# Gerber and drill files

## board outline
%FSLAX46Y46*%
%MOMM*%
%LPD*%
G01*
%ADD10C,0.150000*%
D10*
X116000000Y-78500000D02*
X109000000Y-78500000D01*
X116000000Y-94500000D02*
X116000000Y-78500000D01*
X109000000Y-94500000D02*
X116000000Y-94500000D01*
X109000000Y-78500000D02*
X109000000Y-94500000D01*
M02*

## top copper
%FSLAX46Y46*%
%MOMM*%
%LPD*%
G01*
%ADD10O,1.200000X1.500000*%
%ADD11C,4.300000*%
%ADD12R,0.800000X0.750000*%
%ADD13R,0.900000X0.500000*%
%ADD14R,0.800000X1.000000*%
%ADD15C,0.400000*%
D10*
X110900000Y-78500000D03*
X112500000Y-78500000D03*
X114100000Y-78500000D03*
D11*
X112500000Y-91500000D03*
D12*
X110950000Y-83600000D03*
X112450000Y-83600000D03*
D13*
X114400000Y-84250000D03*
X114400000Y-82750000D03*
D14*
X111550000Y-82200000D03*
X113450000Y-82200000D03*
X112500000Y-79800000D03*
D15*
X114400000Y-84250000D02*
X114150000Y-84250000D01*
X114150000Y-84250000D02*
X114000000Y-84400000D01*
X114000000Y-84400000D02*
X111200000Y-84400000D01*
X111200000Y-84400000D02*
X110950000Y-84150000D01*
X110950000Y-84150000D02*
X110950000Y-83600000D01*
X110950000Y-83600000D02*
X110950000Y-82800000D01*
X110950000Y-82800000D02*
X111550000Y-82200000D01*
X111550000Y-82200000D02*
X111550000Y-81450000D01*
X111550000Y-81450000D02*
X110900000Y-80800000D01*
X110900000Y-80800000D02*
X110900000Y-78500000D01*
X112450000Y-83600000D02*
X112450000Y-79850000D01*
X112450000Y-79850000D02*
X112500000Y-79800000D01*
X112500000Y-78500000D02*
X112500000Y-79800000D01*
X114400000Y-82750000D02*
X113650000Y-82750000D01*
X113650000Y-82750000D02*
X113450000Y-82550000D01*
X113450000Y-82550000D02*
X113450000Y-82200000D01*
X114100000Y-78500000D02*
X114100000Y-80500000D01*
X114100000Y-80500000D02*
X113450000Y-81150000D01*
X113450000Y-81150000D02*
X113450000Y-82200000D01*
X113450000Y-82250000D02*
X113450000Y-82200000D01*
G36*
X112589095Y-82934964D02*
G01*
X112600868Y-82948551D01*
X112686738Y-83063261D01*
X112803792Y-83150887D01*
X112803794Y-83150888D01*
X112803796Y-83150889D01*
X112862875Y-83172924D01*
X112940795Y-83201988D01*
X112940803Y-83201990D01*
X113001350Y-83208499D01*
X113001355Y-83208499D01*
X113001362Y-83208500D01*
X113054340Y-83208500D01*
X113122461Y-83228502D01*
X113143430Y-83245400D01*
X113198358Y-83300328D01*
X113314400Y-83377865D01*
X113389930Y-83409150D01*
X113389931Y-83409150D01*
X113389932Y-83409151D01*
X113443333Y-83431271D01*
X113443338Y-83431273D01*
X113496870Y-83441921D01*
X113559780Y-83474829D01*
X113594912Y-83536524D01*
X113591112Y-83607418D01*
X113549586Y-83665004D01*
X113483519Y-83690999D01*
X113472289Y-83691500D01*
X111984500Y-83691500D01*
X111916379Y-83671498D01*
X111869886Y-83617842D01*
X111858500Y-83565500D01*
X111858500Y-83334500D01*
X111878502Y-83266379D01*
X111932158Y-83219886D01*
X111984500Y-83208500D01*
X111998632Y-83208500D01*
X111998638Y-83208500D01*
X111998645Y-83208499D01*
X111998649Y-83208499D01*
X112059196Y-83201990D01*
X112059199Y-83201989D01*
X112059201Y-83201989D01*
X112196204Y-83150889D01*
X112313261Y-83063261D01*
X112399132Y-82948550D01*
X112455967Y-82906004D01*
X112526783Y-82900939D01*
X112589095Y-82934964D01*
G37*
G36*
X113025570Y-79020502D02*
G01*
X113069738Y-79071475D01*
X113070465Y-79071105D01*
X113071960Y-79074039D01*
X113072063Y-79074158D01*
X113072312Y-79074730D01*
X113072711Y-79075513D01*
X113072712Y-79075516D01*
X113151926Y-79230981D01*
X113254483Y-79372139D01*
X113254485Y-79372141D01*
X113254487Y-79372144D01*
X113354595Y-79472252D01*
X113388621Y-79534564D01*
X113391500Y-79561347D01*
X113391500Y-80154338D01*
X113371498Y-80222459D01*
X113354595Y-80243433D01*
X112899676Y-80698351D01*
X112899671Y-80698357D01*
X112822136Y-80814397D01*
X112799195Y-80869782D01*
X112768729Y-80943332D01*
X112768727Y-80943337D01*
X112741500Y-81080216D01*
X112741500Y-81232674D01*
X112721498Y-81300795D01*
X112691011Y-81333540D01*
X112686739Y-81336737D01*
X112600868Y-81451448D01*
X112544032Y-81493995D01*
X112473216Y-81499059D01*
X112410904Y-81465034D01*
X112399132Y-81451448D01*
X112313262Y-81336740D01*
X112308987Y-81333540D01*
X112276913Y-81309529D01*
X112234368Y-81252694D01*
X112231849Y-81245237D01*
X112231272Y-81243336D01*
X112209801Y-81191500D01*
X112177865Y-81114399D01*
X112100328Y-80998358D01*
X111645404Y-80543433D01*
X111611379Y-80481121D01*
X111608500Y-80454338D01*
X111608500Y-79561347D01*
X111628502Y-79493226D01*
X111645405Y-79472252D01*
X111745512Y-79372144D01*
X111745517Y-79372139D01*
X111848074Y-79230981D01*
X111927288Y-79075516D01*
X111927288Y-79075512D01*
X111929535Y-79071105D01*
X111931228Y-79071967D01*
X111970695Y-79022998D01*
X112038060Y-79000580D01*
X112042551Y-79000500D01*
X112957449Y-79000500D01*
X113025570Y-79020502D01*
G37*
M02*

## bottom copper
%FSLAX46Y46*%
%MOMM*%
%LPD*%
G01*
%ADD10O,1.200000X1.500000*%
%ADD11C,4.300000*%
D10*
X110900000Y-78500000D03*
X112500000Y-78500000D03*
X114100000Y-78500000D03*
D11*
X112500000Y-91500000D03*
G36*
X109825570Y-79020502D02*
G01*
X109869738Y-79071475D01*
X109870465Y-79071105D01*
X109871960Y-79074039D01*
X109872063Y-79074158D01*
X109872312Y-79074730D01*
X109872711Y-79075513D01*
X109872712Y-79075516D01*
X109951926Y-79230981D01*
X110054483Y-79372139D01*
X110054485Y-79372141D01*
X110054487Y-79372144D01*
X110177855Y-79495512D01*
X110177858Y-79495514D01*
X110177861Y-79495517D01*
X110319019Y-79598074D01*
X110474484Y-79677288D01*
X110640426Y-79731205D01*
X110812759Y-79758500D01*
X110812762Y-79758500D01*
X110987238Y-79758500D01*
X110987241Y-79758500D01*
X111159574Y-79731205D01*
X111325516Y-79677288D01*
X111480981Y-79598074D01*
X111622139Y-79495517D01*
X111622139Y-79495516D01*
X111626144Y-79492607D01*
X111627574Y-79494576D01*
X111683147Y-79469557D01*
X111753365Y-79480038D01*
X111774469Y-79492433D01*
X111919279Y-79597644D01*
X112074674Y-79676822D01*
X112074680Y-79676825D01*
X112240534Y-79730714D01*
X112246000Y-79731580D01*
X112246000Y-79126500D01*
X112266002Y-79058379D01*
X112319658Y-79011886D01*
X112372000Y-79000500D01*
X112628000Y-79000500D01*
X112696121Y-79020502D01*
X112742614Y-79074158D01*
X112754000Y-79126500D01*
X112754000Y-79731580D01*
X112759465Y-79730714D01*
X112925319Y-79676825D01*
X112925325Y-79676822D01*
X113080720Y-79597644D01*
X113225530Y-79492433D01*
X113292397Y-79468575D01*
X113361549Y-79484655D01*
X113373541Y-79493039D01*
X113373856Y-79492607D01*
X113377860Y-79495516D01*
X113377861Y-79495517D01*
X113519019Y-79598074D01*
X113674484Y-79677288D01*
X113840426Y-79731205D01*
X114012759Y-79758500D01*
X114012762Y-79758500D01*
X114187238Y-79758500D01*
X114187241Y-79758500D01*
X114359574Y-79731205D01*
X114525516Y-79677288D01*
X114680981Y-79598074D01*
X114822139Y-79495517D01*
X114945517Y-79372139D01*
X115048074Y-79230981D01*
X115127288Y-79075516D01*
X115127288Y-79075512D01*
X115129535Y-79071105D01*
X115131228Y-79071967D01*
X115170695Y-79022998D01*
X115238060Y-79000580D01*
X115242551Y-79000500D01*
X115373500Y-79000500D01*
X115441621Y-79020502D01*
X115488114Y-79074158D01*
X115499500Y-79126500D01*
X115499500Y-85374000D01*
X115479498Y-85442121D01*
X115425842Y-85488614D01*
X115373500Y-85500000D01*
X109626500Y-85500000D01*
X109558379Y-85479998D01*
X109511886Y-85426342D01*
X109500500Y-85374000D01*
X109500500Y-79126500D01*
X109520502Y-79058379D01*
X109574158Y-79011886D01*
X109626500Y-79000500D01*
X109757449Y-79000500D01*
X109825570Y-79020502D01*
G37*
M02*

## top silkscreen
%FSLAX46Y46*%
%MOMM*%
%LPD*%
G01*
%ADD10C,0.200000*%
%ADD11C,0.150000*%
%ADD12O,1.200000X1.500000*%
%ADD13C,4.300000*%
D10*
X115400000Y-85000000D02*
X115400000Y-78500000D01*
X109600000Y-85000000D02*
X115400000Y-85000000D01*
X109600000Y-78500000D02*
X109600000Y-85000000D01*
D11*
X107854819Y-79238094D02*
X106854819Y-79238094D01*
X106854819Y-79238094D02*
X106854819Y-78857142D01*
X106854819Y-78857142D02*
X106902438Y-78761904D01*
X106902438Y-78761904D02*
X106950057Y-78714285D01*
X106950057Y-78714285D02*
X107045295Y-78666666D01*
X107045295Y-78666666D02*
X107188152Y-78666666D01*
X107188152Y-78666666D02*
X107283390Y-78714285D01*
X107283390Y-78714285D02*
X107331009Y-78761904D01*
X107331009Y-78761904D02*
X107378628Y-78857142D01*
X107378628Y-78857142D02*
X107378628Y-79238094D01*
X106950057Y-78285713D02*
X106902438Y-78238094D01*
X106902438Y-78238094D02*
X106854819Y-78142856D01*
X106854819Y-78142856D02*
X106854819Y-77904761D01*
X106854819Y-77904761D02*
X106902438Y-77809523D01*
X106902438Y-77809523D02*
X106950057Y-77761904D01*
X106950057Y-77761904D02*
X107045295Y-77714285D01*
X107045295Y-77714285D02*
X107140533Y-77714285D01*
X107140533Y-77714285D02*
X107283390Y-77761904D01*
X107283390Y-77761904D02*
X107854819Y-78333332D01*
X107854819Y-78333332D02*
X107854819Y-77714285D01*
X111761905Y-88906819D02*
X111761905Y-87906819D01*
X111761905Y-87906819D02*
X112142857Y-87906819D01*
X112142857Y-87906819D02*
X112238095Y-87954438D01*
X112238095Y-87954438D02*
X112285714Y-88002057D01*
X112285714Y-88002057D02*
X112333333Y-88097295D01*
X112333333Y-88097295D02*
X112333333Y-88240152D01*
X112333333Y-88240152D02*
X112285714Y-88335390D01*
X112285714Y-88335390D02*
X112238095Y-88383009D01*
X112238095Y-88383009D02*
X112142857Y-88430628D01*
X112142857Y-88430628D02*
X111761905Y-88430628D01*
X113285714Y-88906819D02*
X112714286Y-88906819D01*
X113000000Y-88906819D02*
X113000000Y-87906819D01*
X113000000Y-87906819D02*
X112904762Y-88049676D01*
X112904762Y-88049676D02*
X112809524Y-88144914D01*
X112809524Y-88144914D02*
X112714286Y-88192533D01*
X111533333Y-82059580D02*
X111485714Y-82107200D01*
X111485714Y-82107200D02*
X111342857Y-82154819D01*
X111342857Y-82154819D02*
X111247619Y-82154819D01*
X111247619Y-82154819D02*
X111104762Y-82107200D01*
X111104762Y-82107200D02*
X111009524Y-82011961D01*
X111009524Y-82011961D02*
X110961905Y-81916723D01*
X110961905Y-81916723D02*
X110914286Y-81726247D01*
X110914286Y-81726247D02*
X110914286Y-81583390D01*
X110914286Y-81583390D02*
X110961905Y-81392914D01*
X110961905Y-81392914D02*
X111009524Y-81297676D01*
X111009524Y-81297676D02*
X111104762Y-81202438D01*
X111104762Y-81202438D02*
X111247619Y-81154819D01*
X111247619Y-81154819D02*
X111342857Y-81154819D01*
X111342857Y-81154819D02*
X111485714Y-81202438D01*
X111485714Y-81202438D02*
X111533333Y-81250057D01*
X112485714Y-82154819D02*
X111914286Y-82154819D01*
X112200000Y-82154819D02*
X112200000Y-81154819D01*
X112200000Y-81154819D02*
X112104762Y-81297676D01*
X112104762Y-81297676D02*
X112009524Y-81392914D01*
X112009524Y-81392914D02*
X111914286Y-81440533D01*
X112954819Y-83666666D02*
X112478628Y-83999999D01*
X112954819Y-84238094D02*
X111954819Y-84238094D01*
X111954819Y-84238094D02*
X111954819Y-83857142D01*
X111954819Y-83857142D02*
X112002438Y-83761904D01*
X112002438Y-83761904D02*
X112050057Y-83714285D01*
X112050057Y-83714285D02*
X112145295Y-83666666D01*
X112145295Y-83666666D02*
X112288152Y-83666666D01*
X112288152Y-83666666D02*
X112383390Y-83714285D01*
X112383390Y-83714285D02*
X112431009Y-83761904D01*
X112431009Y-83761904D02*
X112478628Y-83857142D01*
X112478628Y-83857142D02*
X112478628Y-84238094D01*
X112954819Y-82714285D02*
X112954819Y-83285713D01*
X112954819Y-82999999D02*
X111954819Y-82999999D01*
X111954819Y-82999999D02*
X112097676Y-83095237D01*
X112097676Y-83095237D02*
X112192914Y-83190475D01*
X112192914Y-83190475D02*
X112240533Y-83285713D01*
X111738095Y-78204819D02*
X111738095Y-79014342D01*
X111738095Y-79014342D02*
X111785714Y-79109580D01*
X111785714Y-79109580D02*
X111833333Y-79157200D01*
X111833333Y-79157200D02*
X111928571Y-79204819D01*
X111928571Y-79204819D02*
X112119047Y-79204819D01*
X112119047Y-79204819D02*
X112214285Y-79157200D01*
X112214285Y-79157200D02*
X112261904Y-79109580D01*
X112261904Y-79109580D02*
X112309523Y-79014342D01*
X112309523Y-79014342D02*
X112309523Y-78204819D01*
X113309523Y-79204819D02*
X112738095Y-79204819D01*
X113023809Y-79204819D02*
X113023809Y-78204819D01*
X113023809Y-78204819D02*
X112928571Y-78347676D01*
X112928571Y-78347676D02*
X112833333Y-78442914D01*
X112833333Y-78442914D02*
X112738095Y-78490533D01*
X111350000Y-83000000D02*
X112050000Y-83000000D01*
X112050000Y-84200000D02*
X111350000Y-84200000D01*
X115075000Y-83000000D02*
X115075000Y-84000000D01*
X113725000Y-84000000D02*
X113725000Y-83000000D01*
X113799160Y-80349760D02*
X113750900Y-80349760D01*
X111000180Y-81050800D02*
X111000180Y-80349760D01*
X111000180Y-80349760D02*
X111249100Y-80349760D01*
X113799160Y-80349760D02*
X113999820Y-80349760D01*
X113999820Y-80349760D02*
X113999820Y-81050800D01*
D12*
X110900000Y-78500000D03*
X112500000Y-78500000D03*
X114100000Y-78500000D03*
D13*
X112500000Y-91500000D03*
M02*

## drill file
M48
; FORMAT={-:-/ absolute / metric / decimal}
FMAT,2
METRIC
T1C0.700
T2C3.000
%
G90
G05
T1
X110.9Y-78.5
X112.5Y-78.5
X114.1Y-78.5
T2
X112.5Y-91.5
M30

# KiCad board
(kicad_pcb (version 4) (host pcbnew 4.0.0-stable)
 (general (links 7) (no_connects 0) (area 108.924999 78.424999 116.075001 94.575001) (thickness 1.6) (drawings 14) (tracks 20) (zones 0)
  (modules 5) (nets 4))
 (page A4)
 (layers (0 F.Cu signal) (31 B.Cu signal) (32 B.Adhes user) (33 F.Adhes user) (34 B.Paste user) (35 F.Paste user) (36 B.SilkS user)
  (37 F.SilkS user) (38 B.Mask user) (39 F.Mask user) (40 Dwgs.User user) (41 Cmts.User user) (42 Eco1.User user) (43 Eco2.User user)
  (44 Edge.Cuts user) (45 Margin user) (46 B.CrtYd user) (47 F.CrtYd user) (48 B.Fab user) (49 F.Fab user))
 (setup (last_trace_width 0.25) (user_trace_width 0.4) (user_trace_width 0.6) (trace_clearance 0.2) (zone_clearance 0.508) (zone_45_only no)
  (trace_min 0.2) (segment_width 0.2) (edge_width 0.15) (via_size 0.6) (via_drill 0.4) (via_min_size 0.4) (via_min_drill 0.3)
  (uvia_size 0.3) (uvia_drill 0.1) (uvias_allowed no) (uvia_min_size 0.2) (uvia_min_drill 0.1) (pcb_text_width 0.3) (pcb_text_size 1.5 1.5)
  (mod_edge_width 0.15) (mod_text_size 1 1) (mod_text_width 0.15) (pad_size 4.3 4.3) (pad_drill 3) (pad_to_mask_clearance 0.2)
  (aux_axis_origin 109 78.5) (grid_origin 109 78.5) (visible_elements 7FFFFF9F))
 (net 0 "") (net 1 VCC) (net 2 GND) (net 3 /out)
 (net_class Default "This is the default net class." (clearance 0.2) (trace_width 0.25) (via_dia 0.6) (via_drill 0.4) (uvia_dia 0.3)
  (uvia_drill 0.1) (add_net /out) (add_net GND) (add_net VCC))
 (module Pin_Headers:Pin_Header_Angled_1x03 (layer F.Cu) (at 112.5 78.5 90)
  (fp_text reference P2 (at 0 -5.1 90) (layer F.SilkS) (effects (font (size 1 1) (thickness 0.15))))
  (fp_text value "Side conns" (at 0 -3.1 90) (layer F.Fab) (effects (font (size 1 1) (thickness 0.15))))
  (pad 1 thru_hole oval (at 0 -1.6 90) (size 1.5 1.2) (drill 0.7) (layers *.Cu *.Mask F.SilkS) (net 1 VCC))
  (pad 2 thru_hole oval (at 0 0 90) (size 1.5 1.2) (drill 0.7) (layers *.Cu *.Mask F.SilkS) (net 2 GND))
  (pad 3 thru_hole oval (at 0 1.6 90) (size 1.5 1.2) (drill 0.7) (layers *.Cu *.Mask F.SilkS) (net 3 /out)))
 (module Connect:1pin (layer F.Cu) (at 112.5 91.5)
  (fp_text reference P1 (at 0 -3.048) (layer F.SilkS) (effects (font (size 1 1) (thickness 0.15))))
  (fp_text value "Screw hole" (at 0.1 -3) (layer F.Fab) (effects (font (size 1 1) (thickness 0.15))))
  (pad 1 thru_hole circle (at 0 0) (size 4.3 4.3) (drill 3) (layers *.Cu *.Mask F.SilkS)))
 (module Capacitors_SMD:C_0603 (layer F.Cu) (at 111.7 83.6)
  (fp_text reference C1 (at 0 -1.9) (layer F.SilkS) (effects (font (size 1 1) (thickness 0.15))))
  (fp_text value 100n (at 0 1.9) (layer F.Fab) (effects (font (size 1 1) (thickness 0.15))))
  (fp_line (start -0.35 -0.6) (end 0.35 -0.6) (layer F.SilkS) (width 0.15))
  (fp_line (start 0.35 0.6) (end -0.35 0.6) (layer F.SilkS) (width 0.15))
  (pad 1 smd rect (at -0.75 0) (size 0.8 0.75) (layers F.Cu F.Paste F.Mask) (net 1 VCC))
  (pad 2 smd rect (at 0.75 0) (size 0.8 0.75) (layers F.Cu F.Paste F.Mask) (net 2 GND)))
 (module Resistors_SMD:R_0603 (layer F.Cu) (at 114.4 83.5 90)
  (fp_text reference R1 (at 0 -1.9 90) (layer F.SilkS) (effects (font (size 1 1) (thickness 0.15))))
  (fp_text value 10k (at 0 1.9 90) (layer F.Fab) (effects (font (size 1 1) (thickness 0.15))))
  (fp_line (start 0.5 0.675) (end -0.5 0.675) (layer F.SilkS) (width 0.15))
  (fp_line (start -0.5 -0.675) (end 0.5 -0.675) (layer F.SilkS) (width 0.15))
  (pad 1 smd rect (at -0.75 0 90) (size 0.5 0.9) (layers F.Cu F.Paste F.Mask) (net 1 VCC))
  (pad 2 smd rect (at 0.75 0 90) (size 0.5 0.9) (layers F.Cu F.Paste F.Mask) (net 3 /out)))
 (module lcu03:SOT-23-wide (layer F.Cu) (at 112.5 81)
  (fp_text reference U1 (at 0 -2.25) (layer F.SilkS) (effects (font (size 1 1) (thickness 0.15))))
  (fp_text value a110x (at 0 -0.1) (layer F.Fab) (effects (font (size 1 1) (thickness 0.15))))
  (fp_line (start 1.29916 -0.65024) (end 1.2509 -0.65024) (layer F.SilkS) (width 0.15))
  (fp_line (start -1.49982 0.0508) (end -1.49982 -0.65024) (layer F.SilkS) (width 0.15))
  (fp_line (start -1.49982 -0.65024) (end -1.2509 -0.65024) (layer F.SilkS) (width 0.15))
  (fp_line (start 1.29916 -0.65024) (end 1.49982 -0.65024) (layer F.SilkS) (width 0.15))
  (fp_line (start 1.49982 -0.65024) (end 1.49982 0.0508) (layer F.SilkS) (width 0.15))
  (pad 1 smd rect (at -0.95 1.2) (size 0.8 1) (layers F.Cu F.Paste F.Mask) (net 1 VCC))
  (pad 2 smd rect (at 0.95 1.2) (size 0.8 1) (layers F.Cu F.Paste F.Mask) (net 3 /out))
  (pad 3 smd rect (at 0 -1.2) (size 0.8 1) (layers F.Cu F.Paste F.Mask) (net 2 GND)))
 (gr_line (start 115.4 85) (end 115.4 78.5) (angle 90) (layer F.SilkS) (width 0.2))
 (gr_line (start 109.6 85) (end 115.4 85) (angle 90) (layer F.SilkS) (width 0.2))
 (gr_line (start 109.6 78.5) (end 109.6 85) (angle 90) (layer F.SilkS) (width 0.2))
 (gr_line (start 116 78.5) (end 109 78.5) (angle 90) (layer Edge.Cuts) (width 0.15))
 (gr_line (start 116 94.5) (end 116 78.5) (angle 90) (layer Edge.Cuts) (width 0.15))
 (gr_line (start 109 94.5) (end 116 94.5) (angle 90) (layer Edge.Cuts) (width 0.15))
 (gr_line (start 109 78.5) (end 109 94.5) (angle 90) (layer Edge.Cuts) (width 0.15))
 (segment (start 114.4 84.25) (end 114.15 84.25) (width 0.4) (layer F.Cu) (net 1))
 (segment (start 114.15 84.25) (end 114 84.4) (width 0.4) (layer F.Cu) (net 1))
 (segment (start 114 84.4) (end 111.2 84.4) (width 0.4) (layer F.Cu) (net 1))
 (segment (start 111.2 84.4) (end 110.95 84.15) (width 0.4) (layer F.Cu) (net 1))
 (segment (start 110.95 84.15) (end 110.95 83.6) (width 0.4) (layer F.Cu) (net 1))
 (segment (start 110.95 83.6) (end 110.95 82.8) (width 0.4) (layer F.Cu) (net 1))
 (segment (start 110.95 82.8) (end 111.55 82.2) (width 0.4) (layer F.Cu) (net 1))
 (segment (start 111.55 82.2) (end 111.55 81.45) (width 0.4) (layer F.Cu) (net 1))
 (segment (start 111.55 81.45) (end 110.9 80.8) (width 0.4) (layer F.Cu) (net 1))
 (segment (start 110.9 80.8) (end 110.9 78.5) (width 0.4) (layer F.Cu) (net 1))
 (segment (start 112.45 83.6) (end 112.45 79.85) (width 0.4) (layer F.Cu) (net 2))
 (segment (start 112.45 79.85) (end 112.5 79.8) (width 0.4) (layer F.Cu) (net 2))
 (segment (start 112.5 78.5) (end 112.5 79.8) (width 0.4) (layer F.Cu) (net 2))
 (segment (start 114.4 82.75) (end 113.65 82.75) (width 0.4) (layer F.Cu) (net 3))
 (segment (start 113.65 82.75) (end 113.45 82.55) (width 0.4) (layer F.Cu) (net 3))
 (segment (start 113.45 82.55) (end 113.45 82.2) (width 0.4) (layer F.Cu) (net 3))
 (segment (start 114.1 78.5) (end 114.1 80.5) (width 0.4) (layer F.Cu) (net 3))
 (segment (start 114.1 80.5) (end 113.45 81.15) (width 0.4) (layer F.Cu) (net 3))
 (segment (start 113.45 81.15) (end 113.45 82.2) (width 0.4) (layer F.Cu) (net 3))
 (segment (start 113.45 82.25) (end 113.45 82.2) (width 0.4) (layer F.Cu) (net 3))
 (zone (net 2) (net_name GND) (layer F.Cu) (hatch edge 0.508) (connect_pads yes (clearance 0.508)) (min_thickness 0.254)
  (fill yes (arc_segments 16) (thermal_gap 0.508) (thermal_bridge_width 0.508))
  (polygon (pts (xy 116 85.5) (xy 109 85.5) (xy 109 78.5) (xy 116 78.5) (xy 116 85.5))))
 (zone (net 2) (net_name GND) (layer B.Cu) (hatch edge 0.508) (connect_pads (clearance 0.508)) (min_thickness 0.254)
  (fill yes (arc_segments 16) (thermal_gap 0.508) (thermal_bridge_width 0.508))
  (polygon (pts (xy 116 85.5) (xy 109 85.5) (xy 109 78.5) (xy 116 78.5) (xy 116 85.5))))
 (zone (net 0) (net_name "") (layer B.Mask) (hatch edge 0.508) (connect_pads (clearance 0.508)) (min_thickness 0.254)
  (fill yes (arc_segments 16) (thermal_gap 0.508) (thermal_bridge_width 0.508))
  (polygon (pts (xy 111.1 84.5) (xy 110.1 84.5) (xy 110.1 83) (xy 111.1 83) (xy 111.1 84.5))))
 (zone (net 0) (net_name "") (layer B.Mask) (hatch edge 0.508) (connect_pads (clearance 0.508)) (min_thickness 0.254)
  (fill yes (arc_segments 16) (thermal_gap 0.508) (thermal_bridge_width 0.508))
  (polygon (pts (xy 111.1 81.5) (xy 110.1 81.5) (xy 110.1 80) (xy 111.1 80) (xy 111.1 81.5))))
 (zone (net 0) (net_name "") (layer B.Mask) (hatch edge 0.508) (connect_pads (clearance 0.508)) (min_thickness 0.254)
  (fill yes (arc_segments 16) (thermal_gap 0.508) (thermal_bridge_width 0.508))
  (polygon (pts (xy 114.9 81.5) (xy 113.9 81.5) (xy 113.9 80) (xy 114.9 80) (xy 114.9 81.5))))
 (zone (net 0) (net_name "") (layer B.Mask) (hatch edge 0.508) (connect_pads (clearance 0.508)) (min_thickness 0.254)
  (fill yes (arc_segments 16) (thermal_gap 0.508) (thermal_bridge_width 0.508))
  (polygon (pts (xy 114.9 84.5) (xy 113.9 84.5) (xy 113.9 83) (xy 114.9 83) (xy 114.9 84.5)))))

